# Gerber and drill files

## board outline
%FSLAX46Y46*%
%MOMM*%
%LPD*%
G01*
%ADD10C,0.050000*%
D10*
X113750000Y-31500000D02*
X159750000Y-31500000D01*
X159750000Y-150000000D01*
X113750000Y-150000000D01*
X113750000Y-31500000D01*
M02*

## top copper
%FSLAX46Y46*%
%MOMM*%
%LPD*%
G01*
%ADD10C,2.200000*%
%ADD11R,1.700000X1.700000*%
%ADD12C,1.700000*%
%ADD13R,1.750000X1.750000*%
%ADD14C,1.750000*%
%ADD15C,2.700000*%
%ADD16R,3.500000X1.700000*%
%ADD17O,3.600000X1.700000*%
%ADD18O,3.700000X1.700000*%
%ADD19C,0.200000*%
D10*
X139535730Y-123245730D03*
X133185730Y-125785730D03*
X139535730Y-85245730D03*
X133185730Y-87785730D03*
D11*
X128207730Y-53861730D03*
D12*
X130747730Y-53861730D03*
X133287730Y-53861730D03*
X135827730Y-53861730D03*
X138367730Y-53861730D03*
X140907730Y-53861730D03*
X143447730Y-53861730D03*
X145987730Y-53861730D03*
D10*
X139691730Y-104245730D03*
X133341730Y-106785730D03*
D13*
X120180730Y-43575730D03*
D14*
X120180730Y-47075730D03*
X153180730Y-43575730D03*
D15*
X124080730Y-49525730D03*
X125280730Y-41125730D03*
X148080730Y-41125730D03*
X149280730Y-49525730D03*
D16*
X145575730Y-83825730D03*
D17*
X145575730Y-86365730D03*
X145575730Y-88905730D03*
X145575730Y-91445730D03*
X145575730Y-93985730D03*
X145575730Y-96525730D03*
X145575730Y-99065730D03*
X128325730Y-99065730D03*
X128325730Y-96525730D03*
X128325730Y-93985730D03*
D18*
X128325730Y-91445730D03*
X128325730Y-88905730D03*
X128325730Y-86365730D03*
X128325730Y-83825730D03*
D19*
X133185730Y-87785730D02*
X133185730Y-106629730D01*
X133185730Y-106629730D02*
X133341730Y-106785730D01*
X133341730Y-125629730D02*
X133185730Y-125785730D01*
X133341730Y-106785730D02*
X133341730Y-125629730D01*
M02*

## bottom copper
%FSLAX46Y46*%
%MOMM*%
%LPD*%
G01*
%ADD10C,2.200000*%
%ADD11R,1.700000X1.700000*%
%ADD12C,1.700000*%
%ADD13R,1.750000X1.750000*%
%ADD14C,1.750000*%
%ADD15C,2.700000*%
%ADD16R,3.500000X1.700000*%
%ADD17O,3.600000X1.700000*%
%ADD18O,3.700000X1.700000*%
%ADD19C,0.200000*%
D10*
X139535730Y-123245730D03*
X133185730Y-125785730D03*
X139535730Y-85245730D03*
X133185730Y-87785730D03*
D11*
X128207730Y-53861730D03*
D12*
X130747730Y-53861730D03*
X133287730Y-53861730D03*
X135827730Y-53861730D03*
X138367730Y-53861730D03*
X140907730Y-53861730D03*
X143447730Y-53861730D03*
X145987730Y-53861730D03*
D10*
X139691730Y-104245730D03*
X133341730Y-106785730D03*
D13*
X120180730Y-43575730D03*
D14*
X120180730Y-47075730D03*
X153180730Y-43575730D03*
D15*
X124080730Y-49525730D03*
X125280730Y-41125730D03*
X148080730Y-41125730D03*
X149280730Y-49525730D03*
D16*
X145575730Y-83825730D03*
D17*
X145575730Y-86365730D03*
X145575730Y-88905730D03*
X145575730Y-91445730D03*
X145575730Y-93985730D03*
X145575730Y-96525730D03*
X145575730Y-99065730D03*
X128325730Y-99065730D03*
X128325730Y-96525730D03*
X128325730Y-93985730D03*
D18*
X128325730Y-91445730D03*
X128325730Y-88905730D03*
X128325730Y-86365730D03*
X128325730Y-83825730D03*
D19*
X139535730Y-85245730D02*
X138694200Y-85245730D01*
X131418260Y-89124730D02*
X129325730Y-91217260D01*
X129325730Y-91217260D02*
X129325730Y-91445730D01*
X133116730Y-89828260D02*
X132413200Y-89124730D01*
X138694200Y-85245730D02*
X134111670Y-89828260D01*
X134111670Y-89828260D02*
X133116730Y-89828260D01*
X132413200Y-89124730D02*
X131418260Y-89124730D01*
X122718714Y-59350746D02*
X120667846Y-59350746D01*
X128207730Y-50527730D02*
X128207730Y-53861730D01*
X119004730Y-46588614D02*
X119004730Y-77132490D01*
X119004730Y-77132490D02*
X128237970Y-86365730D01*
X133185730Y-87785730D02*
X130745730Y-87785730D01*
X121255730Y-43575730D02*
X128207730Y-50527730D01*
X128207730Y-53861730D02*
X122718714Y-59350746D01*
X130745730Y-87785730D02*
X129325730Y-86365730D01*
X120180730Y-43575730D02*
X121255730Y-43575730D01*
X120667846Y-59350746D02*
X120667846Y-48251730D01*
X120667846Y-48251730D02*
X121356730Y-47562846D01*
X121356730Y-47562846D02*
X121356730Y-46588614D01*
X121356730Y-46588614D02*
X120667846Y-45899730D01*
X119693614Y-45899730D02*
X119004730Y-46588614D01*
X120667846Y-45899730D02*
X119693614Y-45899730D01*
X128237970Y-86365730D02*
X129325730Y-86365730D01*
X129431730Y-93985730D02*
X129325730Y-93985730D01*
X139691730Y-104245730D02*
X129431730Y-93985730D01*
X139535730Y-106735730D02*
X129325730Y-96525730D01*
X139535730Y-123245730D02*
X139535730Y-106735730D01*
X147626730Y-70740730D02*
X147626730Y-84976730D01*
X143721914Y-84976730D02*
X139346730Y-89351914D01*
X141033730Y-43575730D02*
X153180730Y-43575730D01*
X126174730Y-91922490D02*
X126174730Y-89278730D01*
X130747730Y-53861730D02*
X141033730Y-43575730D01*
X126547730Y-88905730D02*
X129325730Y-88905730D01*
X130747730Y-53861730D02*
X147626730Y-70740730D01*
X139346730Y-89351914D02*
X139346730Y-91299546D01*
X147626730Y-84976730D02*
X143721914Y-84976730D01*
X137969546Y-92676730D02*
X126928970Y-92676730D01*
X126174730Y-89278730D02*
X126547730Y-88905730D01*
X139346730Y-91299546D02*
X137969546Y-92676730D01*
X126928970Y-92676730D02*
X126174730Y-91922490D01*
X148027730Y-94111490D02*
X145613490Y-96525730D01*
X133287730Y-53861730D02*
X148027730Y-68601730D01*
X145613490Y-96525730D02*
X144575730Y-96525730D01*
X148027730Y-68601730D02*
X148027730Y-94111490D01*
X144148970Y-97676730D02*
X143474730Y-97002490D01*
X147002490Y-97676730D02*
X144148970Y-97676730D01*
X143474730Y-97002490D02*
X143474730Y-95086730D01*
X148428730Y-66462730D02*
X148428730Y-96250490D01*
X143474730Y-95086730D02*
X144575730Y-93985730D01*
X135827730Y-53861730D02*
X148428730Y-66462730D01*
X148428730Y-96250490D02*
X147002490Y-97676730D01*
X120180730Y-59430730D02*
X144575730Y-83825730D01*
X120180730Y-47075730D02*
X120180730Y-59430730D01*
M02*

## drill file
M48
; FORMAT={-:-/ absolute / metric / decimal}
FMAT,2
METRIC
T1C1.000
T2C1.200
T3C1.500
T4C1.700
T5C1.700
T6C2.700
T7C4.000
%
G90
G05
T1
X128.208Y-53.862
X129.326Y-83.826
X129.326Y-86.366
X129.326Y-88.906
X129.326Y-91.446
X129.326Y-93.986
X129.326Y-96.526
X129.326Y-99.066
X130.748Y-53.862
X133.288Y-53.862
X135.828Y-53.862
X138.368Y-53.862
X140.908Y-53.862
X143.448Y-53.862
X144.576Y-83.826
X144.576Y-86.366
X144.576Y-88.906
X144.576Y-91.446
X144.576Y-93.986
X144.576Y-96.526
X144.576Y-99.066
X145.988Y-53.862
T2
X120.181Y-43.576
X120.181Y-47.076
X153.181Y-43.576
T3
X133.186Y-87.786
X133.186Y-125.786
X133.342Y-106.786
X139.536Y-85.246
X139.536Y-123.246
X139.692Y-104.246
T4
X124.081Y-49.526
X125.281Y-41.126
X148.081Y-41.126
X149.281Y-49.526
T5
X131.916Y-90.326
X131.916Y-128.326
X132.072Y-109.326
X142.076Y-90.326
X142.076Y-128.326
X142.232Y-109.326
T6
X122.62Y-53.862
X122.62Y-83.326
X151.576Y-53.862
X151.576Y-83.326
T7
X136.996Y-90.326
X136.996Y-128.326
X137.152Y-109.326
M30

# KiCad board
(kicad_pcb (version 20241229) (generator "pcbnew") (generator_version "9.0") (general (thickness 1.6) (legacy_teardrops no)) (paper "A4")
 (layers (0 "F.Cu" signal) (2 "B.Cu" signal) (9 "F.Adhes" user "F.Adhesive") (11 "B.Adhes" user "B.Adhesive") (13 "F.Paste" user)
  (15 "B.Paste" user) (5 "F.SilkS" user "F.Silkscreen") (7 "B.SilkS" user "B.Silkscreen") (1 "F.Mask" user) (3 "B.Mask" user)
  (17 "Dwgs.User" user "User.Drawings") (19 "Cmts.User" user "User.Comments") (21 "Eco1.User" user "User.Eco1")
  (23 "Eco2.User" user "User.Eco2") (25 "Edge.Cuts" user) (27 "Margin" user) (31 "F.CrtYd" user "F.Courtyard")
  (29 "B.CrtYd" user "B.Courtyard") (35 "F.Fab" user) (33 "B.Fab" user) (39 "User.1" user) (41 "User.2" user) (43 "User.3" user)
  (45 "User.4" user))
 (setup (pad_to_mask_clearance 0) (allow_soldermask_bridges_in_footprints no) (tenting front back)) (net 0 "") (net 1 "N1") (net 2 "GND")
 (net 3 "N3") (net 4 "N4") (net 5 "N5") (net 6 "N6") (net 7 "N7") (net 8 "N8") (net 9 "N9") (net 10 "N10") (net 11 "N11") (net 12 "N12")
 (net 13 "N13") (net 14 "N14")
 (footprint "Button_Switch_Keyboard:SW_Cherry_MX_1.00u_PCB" (layer "F.Cu") (at 139.53573 123.24573)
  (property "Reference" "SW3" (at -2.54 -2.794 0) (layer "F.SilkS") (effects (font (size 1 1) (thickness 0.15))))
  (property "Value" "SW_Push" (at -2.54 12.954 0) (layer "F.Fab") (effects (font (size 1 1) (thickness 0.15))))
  (pad "" np_thru_hole circle (at -7.62 5.08) (size 1.7 1.7) (drill 1.7) (layers "*.Cu" "*.Mask"))
  (pad "" np_thru_hole circle (at -2.54 5.08) (size 4 4) (drill 4) (layers "*.Cu" "*.Mask"))
  (pad "" np_thru_hole circle (at 2.54 5.08) (size 1.7 1.7) (drill 1.7) (layers "*.Cu" "*.Mask"))
  (pad "1" thru_hole circle (at 0 0) (size 2.2 2.2) (drill 1.5) (layers "*.Cu" "*.Mask") (remove_unused_layers no) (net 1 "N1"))
  (pad "2" thru_hole circle (at -6.35 2.54) (size 2.2 2.2) (drill 1.5) (layers "*.Cu" "*.Mask") (remove_unused_layers no) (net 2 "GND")))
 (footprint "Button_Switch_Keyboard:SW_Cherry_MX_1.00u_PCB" (layer "F.Cu") (at 139.53573 85.24573)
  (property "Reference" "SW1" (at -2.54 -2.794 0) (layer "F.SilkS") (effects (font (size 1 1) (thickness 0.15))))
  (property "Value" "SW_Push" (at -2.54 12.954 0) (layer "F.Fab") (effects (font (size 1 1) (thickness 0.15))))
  (pad "" np_thru_hole circle (at -7.62 5.08) (size 1.7 1.7) (drill 1.7) (layers "*.Cu" "*.Mask"))
  (pad "" np_thru_hole circle (at -2.54 5.08) (size 4 4) (drill 4) (layers "*.Cu" "*.Mask"))
  (pad "" np_thru_hole circle (at 2.54 5.08) (size 1.7 1.7) (drill 1.7) (layers "*.Cu" "*.Mask"))
  (pad "1" thru_hole circle (at 0 0) (size 2.2 2.2) (drill 1.5) (layers "*.Cu" "*.Mask") (remove_unused_layers no) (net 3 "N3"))
  (pad "2" thru_hole circle (at -6.35 2.54) (size 2.2 2.2) (drill 1.5) (layers "*.Cu" "*.Mask") (remove_unused_layers no) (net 2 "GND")))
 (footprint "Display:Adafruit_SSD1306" (layer "F.Cu") (at 128.20773 53.86173)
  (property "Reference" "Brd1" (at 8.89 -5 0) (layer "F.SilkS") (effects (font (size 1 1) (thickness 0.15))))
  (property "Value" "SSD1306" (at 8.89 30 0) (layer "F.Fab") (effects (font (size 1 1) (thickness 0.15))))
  (pad "" np_thru_hole circle (at -5.588 0) (size 2.7 2.7) (drill 2.7) (layers "*.Cu" "*.Mask"))
  (pad "" np_thru_hole circle (at -5.588 29.464) (size 2.7 2.7) (drill 2.7) (layers "*.Cu" "*.Mask"))
  (pad "" np_thru_hole circle (at 23.368 0) (size 2.7 2.7) (drill 2.7) (layers "*.Cu" "*.Mask"))
  (pad "" np_thru_hole circle (at 23.368 29.464) (size 2.7 2.7) (drill 2.7) (layers "*.Cu" "*.Mask"))
  (pad "1" thru_hole rect (at 0 0) (size 1.7 1.7) (drill 1) (layers "*.Cu" "*.Mask") (remove_unused_layers no) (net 2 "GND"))
  (pad "2" thru_hole circle (at 2.54 0) (size 1.7 1.7) (drill 1) (layers "*.Cu" "*.Mask") (remove_unused_layers no) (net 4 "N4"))
  (pad "3" thru_hole circle (at 5.08 0) (size 1.7 1.7) (drill 1) (layers "*.Cu" "*.Mask") (remove_unused_layers no) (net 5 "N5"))
  (pad "4" thru_hole circle (at 7.62 0) (size 1.7 1.7) (drill 1) (layers "*.Cu" "*.Mask") (remove_unused_layers no) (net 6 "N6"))
  (pad "5" thru_hole circle (at 10.16 0) (size 1.7 1.7) (drill 1) (layers "*.Cu" "*.Mask") (remove_unused_layers no))
  (pad "6" thru_hole circle (at 12.7 0) (size 1.7 1.7) (drill 1) (layers "*.Cu" "*.Mask") (remove_unused_layers no))
  (pad "7" thru_hole circle (at 15.24 0) (size 1.7 1.7) (drill 1) (layers "*.Cu" "*.Mask") (remove_unused_layers no))
  (pad "8" thru_hole circle (at 17.78 0) (size 1.7 1.7) (drill 1) (layers "*.Cu" "*.Mask") (remove_unused_layers no)))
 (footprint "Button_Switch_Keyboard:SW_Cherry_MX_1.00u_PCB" (layer "F.Cu") (at 139.69173 104.24573)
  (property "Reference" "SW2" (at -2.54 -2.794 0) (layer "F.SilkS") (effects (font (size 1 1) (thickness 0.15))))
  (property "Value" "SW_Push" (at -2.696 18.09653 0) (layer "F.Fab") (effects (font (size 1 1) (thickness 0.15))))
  (pad "" np_thru_hole circle (at -7.62 5.08) (size 1.7 1.7) (drill 1.7) (layers "*.Cu" "*.Mask"))
  (pad "" np_thru_hole circle (at -2.54 5.08) (size 4 4) (drill 4) (layers "*.Cu" "*.Mask"))
  (pad "" np_thru_hole circle (at 2.54 5.08) (size 1.7 1.7) (drill 1.7) (layers "*.Cu" "*.Mask"))
  (pad "1" thru_hole circle (at 0 0) (size 2.2 2.2) (drill 1.5) (layers "*.Cu" "*.Mask") (remove_unused_layers no) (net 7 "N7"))
  (pad "2" thru_hole circle (at -6.35 2.54) (size 2.2 2.2) (drill 1.5) (layers "*.Cu" "*.Mask") (remove_unused_layers no) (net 2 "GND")))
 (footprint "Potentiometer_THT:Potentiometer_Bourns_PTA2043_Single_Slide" (layer "F.Cu") (at 120.18073 43.57573)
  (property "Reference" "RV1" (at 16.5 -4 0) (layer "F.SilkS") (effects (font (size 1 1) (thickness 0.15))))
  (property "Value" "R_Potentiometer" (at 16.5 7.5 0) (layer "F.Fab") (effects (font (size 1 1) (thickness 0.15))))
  (pad "1" thru_hole rect (at 0 0) (size 1.75 1.75) (drill 1.2) (layers "*.Cu" "*.Mask") (remove_unused_layers no) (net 2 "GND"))
  (pad "2" thru_hole circle (at 0 3.5) (size 1.75 1.75) (drill 1.2) (layers "*.Cu" "*.Mask") (remove_unused_layers no) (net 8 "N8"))
  (pad "3" thru_hole circle (at 33 0) (size 1.75 1.75) (drill 1.2) (layers "*.Cu" "*.Mask") (remove_unused_layers no) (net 4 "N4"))
  (pad "MP" thru_hole circle (at 3.9 5.95) (size 2.7 2.7) (drill 1.7) (layers "*.Cu" "*.Mask") (remove_unused_layers no))
  (pad "MP" thru_hole circle (at 5.1 -2.45) (size 2.7 2.7) (drill 1.7) (layers "*.Cu" "*.Mask") (remove_unused_layers no))
  (pad "MP" thru_hole circle (at 27.9 -2.45) (size 2.7 2.7) (drill 1.7) (layers "*.Cu" "*.Mask") (remove_unused_layers no))
  (pad "MP" thru_hole circle (at 29.1 5.95) (size 2.7 2.7) (drill 1.7) (layers "*.Cu" "*.Mask") (remove_unused_layers no)))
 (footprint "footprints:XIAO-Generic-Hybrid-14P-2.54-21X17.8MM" (layer "B.Cu") (at 136.95073 91.44573 180)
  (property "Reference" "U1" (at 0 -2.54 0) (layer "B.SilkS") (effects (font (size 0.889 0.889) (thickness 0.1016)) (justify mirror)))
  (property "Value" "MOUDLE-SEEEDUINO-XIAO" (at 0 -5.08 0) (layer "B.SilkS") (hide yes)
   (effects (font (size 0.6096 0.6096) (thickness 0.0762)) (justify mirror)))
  (pad "1" thru_hole rect (at -7.625 7.62 180) (size 3.5 1.7) (drill 1 (offset -1 0)) (layers "*.Cu" "*.Mask") (remove_unused_layers no)
   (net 8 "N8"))
  (pad "2" thru_hole oval (at -7.625 5.08 180) (size 3.6 1.7) (drill 1 (offset -1 0)) (layers "*.Cu" "*.Mask") (remove_unused_layers no)
   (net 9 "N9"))
  (pad "3" thru_hole oval (at -7.625 2.54 180) (size 3.6 1.7) (drill 1 (offset -1 0)) (layers "*.Cu" "*.Mask") (remove_unused_layers no)
   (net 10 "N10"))
  (pad "4" thru_hole oval (at -7.625 0 180) (size 3.6 1.7) (drill 1 (offset -1 0)) (layers "*.Cu" "*.Mask") (remove_unused_layers no)
   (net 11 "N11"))
  (pad "5" thru_hole oval (at -7.625 -2.54 180) (size 3.6 1.7) (drill 1 (offset -1 0)) (layers "*.Cu" "*.Mask") (remove_unused_layers no)
   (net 6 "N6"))
  (pad "6" thru_hole oval (at -7.625 -5.08) (size 3.6 1.7) (drill 1 (offset 1 0)) (layers "*.Cu" "*.Mask") (remove_unused_layers no)
   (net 5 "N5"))
  (pad "7" thru_hole oval (at -7.625 -7.62 180) (size 3.6 1.7) (drill 1 (offset -1 0)) (layers "*.Cu" "*.Mask") (remove_unused_layers no)
   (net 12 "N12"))
  (pad "8" thru_hole oval (at 7.625 -7.62 180) (size 3.6 1.7) (drill 1 (offset 1 0)) (layers "*.Cu" "*.Mask") (remove_unused_layers no)
   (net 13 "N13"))
  (pad "9" thru_hole oval (at 7.625 -5.08 180) (size 3.6 1.7) (drill 1 (offset 1 0)) (layers "*.Cu" "*.Mask") (remove_unused_layers no)
   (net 1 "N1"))
  (pad "10" thru_hole oval (at 7.625 -2.54 180) (size 3.6 1.7) (drill 1 (offset 1 0)) (layers "*.Cu" "*.Mask") (remove_unused_layers no)
   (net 7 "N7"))
  (pad "11" thru_hole oval (at 7.625 0 180) (size 3.7 1.7) (drill 1 (offset 1 0)) (layers "*.Cu" "*.Mask") (remove_unused_layers no)
   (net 3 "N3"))
  (pad "12" thru_hole oval (at 7.625 2.54 180) (size 3.7 1.7) (drill 1 (offset 1 0)) (layers "*.Cu" "*.Mask") (remove_unused_layers no)
   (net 4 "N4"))
  (pad "13" thru_hole oval (at 7.625 5.08 180) (size 3.7 1.7) (drill 1 (offset 1 0)) (layers "*.Cu" "*.Mask") (remove_unused_layers no)
   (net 2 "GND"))
  (pad "14" thru_hole oval (at 7.625 7.62 180) (size 3.7 1.7) (drill 1 (offset 1 0)) (layers "*.Cu" "*.Mask") (remove_unused_layers no)
   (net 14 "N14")))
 (gr_rect (start 113.75 31.5) (end 159.75 150) (stroke (width 0.05) (type default)) (fill no) (layer "Edge.Cuts"))
 (segment (start 139.53573 85.24573) (end 138.6942 85.24573) (width 0.2) (layer "B.Cu") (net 3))
 (segment (start 131.41826 89.12473) (end 129.32573 91.21726) (width 0.2) (layer "B.Cu") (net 3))
 (segment (start 129.32573 91.21726) (end 129.32573 91.44573) (width 0.2) (layer "B.Cu") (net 3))
 (segment (start 133.11673 89.82826) (end 132.4132 89.12473) (width 0.2) (layer "B.Cu") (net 3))
 (segment (start 138.6942 85.24573) (end 134.11167 89.82826) (width 0.2) (layer "B.Cu") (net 3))
 (segment (start 134.11167 89.82826) (end 133.11673 89.82826) (width 0.2) (layer "B.Cu") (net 3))
 (segment (start 132.4132 89.12473) (end 131.41826 89.12473) (width 0.2) (layer "B.Cu") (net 3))
 (segment (start 133.18573 87.78573) (end 133.18573 106.62973) (width 0.2) (layer "F.Cu") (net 2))
 (segment (start 133.18573 106.62973) (end 133.34173 106.78573) (width 0.2) (layer "F.Cu") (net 2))
 (segment (start 133.34173 125.62973) (end 133.18573 125.78573) (width 0.2) (layer "F.Cu") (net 2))
 (segment (start 133.34173 106.78573) (end 133.34173 125.62973) (width 0.2) (layer "F.Cu") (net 2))
 (segment (start 122.718714 59.350746) (end 120.667846 59.350746) (width 0.2) (layer "B.Cu") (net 2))
 (segment (start 128.20773 50.52773) (end 128.20773 53.86173) (width 0.2) (layer "B.Cu") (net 2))
 (segment (start 119.00473 46.588614) (end 119.00473 77.13249) (width 0.2) (layer "B.Cu") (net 2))
 (segment (start 119.00473 77.13249) (end 128.23797 86.36573) (width 0.2) (layer "B.Cu") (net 2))
 (segment (start 133.18573 87.78573) (end 130.74573 87.78573) (width 0.2) (layer "B.Cu") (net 2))
 (segment (start 121.25573 43.57573) (end 128.20773 50.52773) (width 0.2) (layer "B.Cu") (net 2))
 (segment (start 128.20773 53.86173) (end 122.718714 59.350746) (width 0.2) (layer "B.Cu") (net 2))
 (segment (start 130.74573 87.78573) (end 129.32573 86.36573) (width 0.2) (layer "B.Cu") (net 2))
 (segment (start 120.18073 43.57573) (end 121.25573 43.57573) (width 0.2) (layer "B.Cu") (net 2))
 (segment (start 120.667846 59.350746) (end 120.667846 48.25173) (width 0.2) (layer "B.Cu") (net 2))
 (segment (start 120.667846 48.25173) (end 121.35673 47.562846) (width 0.2) (layer "B.Cu") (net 2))
 (segment (start 121.35673 47.562846) (end 121.35673 46.588614) (width 0.2) (layer "B.Cu") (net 2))
 (segment (start 121.35673 46.588614) (end 120.667846 45.89973) (width 0.2) (layer "B.Cu") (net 2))
 (segment (start 119.693614 45.89973) (end 119.00473 46.588614) (width 0.2) (layer "B.Cu") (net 2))
 (segment (start 120.667846 45.89973) (end 119.693614 45.89973) (width 0.2) (layer "B.Cu") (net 2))
 (segment (start 128.23797 86.36573) (end 129.32573 86.36573) (width 0.2) (layer "B.Cu") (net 2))
 (segment (start 129.43173 93.98573) (end 129.32573 93.98573) (width 0.2) (layer "B.Cu") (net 7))
 (segment (start 139.69173 104.24573) (end 129.43173 93.98573) (width 0.2) (layer "B.Cu") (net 7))
 (segment (start 139.53573 106.73573) (end 129.32573 96.52573) (width 0.2) (layer "B.Cu") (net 1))
 (segment (start 139.53573 123.24573) (end 139.53573 106.73573) (width 0.2) (layer "B.Cu") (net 1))
 (segment (start 147.62673 70.74073) (end 147.62673 84.97673) (width 0.2) (layer "B.Cu") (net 4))
 (segment (start 143.721914 84.97673) (end 139.34673 89.351914) (width 0.2) (layer "B.Cu") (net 4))
 (segment (start 141.03373 43.57573) (end 153.18073 43.57573) (width 0.2) (layer "B.Cu") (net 4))
 (segment (start 126.17473 91.92249) (end 126.17473 89.27873) (width 0.2) (layer "B.Cu") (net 4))
 (segment (start 130.74773 53.86173) (end 141.03373 43.57573) (width 0.2) (layer "B.Cu") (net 4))
 (segment (start 126.54773 88.90573) (end 129.32573 88.90573) (width 0.2) (layer "B.Cu") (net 4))
 (segment (start 130.74773 53.86173) (end 147.62673 70.74073) (width 0.2) (layer "B.Cu") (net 4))
 (segment (start 139.34673 89.351914) (end 139.34673 91.299546) (width 0.2) (layer "B.Cu") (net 4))
 (segment (start 147.62673 84.97673) (end 143.721914 84.97673) (width 0.2) (layer "B.Cu") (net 4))
 (segment (start 137.969546 92.67673) (end 126.92897 92.67673) (width 0.2) (layer "B.Cu") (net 4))
 (segment (start 126.17473 89.27873) (end 126.54773 88.90573) (width 0.2) (layer "B.Cu") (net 4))
 (segment (start 139.34673 91.299546) (end 137.969546 92.67673) (width 0.2) (layer "B.Cu") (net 4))
 (segment (start 126.92897 92.67673) (end 126.17473 91.92249) (width 0.2) (layer "B.Cu") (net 4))
 (segment (start 148.02773 94.11149) (end 145.61349 96.52573) (width 0.2) (layer "B.Cu") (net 5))
 (segment (start 133.28773 53.86173) (end 148.02773 68.60173) (width 0.2) (layer "B.Cu") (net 5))
 (segment (start 145.61349 96.52573) (end 144.57573 96.52573) (width 0.2) (layer "B.Cu") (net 5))
 (segment (start 148.02773 68.60173) (end 148.02773 94.11149) (width 0.2) (layer "B.Cu") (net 5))
 (segment (start 144.14897 97.67673) (end 143.47473 97.00249) (width 0.2) (layer "B.Cu") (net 6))
 (segment (start 147.00249 97.67673) (end 144.14897 97.67673) (width 0.2) (layer "B.Cu") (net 6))
 (segment (start 143.47473 97.00249) (end 143.47473 95.08673) (width 0.2) (layer "B.Cu") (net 6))
 (segment (start 148.42873 66.46273) (end 148.42873 96.25049) (width 0.2) (layer "B.Cu") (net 6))
 (segment (start 143.47473 95.08673) (end 144.57573 93.98573) (width 0.2) (layer "B.Cu") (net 6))
 (segment (start 135.82773 53.86173) (end 148.42873 66.46273) (width 0.2) (layer "B.Cu") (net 6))
 (segment (start 148.42873 96.25049) (end 147.00249 97.67673) (width 0.2) (layer "B.Cu") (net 6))
 (segment (start 120.18073 59.43073) (end 144.57573 83.82573) (width 0.2) (layer "B.Cu") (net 8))
 (segment (start 120.18073 47.07573) (end 120.18073 59.43073) (width 0.2) (layer "B.Cu") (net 8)))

